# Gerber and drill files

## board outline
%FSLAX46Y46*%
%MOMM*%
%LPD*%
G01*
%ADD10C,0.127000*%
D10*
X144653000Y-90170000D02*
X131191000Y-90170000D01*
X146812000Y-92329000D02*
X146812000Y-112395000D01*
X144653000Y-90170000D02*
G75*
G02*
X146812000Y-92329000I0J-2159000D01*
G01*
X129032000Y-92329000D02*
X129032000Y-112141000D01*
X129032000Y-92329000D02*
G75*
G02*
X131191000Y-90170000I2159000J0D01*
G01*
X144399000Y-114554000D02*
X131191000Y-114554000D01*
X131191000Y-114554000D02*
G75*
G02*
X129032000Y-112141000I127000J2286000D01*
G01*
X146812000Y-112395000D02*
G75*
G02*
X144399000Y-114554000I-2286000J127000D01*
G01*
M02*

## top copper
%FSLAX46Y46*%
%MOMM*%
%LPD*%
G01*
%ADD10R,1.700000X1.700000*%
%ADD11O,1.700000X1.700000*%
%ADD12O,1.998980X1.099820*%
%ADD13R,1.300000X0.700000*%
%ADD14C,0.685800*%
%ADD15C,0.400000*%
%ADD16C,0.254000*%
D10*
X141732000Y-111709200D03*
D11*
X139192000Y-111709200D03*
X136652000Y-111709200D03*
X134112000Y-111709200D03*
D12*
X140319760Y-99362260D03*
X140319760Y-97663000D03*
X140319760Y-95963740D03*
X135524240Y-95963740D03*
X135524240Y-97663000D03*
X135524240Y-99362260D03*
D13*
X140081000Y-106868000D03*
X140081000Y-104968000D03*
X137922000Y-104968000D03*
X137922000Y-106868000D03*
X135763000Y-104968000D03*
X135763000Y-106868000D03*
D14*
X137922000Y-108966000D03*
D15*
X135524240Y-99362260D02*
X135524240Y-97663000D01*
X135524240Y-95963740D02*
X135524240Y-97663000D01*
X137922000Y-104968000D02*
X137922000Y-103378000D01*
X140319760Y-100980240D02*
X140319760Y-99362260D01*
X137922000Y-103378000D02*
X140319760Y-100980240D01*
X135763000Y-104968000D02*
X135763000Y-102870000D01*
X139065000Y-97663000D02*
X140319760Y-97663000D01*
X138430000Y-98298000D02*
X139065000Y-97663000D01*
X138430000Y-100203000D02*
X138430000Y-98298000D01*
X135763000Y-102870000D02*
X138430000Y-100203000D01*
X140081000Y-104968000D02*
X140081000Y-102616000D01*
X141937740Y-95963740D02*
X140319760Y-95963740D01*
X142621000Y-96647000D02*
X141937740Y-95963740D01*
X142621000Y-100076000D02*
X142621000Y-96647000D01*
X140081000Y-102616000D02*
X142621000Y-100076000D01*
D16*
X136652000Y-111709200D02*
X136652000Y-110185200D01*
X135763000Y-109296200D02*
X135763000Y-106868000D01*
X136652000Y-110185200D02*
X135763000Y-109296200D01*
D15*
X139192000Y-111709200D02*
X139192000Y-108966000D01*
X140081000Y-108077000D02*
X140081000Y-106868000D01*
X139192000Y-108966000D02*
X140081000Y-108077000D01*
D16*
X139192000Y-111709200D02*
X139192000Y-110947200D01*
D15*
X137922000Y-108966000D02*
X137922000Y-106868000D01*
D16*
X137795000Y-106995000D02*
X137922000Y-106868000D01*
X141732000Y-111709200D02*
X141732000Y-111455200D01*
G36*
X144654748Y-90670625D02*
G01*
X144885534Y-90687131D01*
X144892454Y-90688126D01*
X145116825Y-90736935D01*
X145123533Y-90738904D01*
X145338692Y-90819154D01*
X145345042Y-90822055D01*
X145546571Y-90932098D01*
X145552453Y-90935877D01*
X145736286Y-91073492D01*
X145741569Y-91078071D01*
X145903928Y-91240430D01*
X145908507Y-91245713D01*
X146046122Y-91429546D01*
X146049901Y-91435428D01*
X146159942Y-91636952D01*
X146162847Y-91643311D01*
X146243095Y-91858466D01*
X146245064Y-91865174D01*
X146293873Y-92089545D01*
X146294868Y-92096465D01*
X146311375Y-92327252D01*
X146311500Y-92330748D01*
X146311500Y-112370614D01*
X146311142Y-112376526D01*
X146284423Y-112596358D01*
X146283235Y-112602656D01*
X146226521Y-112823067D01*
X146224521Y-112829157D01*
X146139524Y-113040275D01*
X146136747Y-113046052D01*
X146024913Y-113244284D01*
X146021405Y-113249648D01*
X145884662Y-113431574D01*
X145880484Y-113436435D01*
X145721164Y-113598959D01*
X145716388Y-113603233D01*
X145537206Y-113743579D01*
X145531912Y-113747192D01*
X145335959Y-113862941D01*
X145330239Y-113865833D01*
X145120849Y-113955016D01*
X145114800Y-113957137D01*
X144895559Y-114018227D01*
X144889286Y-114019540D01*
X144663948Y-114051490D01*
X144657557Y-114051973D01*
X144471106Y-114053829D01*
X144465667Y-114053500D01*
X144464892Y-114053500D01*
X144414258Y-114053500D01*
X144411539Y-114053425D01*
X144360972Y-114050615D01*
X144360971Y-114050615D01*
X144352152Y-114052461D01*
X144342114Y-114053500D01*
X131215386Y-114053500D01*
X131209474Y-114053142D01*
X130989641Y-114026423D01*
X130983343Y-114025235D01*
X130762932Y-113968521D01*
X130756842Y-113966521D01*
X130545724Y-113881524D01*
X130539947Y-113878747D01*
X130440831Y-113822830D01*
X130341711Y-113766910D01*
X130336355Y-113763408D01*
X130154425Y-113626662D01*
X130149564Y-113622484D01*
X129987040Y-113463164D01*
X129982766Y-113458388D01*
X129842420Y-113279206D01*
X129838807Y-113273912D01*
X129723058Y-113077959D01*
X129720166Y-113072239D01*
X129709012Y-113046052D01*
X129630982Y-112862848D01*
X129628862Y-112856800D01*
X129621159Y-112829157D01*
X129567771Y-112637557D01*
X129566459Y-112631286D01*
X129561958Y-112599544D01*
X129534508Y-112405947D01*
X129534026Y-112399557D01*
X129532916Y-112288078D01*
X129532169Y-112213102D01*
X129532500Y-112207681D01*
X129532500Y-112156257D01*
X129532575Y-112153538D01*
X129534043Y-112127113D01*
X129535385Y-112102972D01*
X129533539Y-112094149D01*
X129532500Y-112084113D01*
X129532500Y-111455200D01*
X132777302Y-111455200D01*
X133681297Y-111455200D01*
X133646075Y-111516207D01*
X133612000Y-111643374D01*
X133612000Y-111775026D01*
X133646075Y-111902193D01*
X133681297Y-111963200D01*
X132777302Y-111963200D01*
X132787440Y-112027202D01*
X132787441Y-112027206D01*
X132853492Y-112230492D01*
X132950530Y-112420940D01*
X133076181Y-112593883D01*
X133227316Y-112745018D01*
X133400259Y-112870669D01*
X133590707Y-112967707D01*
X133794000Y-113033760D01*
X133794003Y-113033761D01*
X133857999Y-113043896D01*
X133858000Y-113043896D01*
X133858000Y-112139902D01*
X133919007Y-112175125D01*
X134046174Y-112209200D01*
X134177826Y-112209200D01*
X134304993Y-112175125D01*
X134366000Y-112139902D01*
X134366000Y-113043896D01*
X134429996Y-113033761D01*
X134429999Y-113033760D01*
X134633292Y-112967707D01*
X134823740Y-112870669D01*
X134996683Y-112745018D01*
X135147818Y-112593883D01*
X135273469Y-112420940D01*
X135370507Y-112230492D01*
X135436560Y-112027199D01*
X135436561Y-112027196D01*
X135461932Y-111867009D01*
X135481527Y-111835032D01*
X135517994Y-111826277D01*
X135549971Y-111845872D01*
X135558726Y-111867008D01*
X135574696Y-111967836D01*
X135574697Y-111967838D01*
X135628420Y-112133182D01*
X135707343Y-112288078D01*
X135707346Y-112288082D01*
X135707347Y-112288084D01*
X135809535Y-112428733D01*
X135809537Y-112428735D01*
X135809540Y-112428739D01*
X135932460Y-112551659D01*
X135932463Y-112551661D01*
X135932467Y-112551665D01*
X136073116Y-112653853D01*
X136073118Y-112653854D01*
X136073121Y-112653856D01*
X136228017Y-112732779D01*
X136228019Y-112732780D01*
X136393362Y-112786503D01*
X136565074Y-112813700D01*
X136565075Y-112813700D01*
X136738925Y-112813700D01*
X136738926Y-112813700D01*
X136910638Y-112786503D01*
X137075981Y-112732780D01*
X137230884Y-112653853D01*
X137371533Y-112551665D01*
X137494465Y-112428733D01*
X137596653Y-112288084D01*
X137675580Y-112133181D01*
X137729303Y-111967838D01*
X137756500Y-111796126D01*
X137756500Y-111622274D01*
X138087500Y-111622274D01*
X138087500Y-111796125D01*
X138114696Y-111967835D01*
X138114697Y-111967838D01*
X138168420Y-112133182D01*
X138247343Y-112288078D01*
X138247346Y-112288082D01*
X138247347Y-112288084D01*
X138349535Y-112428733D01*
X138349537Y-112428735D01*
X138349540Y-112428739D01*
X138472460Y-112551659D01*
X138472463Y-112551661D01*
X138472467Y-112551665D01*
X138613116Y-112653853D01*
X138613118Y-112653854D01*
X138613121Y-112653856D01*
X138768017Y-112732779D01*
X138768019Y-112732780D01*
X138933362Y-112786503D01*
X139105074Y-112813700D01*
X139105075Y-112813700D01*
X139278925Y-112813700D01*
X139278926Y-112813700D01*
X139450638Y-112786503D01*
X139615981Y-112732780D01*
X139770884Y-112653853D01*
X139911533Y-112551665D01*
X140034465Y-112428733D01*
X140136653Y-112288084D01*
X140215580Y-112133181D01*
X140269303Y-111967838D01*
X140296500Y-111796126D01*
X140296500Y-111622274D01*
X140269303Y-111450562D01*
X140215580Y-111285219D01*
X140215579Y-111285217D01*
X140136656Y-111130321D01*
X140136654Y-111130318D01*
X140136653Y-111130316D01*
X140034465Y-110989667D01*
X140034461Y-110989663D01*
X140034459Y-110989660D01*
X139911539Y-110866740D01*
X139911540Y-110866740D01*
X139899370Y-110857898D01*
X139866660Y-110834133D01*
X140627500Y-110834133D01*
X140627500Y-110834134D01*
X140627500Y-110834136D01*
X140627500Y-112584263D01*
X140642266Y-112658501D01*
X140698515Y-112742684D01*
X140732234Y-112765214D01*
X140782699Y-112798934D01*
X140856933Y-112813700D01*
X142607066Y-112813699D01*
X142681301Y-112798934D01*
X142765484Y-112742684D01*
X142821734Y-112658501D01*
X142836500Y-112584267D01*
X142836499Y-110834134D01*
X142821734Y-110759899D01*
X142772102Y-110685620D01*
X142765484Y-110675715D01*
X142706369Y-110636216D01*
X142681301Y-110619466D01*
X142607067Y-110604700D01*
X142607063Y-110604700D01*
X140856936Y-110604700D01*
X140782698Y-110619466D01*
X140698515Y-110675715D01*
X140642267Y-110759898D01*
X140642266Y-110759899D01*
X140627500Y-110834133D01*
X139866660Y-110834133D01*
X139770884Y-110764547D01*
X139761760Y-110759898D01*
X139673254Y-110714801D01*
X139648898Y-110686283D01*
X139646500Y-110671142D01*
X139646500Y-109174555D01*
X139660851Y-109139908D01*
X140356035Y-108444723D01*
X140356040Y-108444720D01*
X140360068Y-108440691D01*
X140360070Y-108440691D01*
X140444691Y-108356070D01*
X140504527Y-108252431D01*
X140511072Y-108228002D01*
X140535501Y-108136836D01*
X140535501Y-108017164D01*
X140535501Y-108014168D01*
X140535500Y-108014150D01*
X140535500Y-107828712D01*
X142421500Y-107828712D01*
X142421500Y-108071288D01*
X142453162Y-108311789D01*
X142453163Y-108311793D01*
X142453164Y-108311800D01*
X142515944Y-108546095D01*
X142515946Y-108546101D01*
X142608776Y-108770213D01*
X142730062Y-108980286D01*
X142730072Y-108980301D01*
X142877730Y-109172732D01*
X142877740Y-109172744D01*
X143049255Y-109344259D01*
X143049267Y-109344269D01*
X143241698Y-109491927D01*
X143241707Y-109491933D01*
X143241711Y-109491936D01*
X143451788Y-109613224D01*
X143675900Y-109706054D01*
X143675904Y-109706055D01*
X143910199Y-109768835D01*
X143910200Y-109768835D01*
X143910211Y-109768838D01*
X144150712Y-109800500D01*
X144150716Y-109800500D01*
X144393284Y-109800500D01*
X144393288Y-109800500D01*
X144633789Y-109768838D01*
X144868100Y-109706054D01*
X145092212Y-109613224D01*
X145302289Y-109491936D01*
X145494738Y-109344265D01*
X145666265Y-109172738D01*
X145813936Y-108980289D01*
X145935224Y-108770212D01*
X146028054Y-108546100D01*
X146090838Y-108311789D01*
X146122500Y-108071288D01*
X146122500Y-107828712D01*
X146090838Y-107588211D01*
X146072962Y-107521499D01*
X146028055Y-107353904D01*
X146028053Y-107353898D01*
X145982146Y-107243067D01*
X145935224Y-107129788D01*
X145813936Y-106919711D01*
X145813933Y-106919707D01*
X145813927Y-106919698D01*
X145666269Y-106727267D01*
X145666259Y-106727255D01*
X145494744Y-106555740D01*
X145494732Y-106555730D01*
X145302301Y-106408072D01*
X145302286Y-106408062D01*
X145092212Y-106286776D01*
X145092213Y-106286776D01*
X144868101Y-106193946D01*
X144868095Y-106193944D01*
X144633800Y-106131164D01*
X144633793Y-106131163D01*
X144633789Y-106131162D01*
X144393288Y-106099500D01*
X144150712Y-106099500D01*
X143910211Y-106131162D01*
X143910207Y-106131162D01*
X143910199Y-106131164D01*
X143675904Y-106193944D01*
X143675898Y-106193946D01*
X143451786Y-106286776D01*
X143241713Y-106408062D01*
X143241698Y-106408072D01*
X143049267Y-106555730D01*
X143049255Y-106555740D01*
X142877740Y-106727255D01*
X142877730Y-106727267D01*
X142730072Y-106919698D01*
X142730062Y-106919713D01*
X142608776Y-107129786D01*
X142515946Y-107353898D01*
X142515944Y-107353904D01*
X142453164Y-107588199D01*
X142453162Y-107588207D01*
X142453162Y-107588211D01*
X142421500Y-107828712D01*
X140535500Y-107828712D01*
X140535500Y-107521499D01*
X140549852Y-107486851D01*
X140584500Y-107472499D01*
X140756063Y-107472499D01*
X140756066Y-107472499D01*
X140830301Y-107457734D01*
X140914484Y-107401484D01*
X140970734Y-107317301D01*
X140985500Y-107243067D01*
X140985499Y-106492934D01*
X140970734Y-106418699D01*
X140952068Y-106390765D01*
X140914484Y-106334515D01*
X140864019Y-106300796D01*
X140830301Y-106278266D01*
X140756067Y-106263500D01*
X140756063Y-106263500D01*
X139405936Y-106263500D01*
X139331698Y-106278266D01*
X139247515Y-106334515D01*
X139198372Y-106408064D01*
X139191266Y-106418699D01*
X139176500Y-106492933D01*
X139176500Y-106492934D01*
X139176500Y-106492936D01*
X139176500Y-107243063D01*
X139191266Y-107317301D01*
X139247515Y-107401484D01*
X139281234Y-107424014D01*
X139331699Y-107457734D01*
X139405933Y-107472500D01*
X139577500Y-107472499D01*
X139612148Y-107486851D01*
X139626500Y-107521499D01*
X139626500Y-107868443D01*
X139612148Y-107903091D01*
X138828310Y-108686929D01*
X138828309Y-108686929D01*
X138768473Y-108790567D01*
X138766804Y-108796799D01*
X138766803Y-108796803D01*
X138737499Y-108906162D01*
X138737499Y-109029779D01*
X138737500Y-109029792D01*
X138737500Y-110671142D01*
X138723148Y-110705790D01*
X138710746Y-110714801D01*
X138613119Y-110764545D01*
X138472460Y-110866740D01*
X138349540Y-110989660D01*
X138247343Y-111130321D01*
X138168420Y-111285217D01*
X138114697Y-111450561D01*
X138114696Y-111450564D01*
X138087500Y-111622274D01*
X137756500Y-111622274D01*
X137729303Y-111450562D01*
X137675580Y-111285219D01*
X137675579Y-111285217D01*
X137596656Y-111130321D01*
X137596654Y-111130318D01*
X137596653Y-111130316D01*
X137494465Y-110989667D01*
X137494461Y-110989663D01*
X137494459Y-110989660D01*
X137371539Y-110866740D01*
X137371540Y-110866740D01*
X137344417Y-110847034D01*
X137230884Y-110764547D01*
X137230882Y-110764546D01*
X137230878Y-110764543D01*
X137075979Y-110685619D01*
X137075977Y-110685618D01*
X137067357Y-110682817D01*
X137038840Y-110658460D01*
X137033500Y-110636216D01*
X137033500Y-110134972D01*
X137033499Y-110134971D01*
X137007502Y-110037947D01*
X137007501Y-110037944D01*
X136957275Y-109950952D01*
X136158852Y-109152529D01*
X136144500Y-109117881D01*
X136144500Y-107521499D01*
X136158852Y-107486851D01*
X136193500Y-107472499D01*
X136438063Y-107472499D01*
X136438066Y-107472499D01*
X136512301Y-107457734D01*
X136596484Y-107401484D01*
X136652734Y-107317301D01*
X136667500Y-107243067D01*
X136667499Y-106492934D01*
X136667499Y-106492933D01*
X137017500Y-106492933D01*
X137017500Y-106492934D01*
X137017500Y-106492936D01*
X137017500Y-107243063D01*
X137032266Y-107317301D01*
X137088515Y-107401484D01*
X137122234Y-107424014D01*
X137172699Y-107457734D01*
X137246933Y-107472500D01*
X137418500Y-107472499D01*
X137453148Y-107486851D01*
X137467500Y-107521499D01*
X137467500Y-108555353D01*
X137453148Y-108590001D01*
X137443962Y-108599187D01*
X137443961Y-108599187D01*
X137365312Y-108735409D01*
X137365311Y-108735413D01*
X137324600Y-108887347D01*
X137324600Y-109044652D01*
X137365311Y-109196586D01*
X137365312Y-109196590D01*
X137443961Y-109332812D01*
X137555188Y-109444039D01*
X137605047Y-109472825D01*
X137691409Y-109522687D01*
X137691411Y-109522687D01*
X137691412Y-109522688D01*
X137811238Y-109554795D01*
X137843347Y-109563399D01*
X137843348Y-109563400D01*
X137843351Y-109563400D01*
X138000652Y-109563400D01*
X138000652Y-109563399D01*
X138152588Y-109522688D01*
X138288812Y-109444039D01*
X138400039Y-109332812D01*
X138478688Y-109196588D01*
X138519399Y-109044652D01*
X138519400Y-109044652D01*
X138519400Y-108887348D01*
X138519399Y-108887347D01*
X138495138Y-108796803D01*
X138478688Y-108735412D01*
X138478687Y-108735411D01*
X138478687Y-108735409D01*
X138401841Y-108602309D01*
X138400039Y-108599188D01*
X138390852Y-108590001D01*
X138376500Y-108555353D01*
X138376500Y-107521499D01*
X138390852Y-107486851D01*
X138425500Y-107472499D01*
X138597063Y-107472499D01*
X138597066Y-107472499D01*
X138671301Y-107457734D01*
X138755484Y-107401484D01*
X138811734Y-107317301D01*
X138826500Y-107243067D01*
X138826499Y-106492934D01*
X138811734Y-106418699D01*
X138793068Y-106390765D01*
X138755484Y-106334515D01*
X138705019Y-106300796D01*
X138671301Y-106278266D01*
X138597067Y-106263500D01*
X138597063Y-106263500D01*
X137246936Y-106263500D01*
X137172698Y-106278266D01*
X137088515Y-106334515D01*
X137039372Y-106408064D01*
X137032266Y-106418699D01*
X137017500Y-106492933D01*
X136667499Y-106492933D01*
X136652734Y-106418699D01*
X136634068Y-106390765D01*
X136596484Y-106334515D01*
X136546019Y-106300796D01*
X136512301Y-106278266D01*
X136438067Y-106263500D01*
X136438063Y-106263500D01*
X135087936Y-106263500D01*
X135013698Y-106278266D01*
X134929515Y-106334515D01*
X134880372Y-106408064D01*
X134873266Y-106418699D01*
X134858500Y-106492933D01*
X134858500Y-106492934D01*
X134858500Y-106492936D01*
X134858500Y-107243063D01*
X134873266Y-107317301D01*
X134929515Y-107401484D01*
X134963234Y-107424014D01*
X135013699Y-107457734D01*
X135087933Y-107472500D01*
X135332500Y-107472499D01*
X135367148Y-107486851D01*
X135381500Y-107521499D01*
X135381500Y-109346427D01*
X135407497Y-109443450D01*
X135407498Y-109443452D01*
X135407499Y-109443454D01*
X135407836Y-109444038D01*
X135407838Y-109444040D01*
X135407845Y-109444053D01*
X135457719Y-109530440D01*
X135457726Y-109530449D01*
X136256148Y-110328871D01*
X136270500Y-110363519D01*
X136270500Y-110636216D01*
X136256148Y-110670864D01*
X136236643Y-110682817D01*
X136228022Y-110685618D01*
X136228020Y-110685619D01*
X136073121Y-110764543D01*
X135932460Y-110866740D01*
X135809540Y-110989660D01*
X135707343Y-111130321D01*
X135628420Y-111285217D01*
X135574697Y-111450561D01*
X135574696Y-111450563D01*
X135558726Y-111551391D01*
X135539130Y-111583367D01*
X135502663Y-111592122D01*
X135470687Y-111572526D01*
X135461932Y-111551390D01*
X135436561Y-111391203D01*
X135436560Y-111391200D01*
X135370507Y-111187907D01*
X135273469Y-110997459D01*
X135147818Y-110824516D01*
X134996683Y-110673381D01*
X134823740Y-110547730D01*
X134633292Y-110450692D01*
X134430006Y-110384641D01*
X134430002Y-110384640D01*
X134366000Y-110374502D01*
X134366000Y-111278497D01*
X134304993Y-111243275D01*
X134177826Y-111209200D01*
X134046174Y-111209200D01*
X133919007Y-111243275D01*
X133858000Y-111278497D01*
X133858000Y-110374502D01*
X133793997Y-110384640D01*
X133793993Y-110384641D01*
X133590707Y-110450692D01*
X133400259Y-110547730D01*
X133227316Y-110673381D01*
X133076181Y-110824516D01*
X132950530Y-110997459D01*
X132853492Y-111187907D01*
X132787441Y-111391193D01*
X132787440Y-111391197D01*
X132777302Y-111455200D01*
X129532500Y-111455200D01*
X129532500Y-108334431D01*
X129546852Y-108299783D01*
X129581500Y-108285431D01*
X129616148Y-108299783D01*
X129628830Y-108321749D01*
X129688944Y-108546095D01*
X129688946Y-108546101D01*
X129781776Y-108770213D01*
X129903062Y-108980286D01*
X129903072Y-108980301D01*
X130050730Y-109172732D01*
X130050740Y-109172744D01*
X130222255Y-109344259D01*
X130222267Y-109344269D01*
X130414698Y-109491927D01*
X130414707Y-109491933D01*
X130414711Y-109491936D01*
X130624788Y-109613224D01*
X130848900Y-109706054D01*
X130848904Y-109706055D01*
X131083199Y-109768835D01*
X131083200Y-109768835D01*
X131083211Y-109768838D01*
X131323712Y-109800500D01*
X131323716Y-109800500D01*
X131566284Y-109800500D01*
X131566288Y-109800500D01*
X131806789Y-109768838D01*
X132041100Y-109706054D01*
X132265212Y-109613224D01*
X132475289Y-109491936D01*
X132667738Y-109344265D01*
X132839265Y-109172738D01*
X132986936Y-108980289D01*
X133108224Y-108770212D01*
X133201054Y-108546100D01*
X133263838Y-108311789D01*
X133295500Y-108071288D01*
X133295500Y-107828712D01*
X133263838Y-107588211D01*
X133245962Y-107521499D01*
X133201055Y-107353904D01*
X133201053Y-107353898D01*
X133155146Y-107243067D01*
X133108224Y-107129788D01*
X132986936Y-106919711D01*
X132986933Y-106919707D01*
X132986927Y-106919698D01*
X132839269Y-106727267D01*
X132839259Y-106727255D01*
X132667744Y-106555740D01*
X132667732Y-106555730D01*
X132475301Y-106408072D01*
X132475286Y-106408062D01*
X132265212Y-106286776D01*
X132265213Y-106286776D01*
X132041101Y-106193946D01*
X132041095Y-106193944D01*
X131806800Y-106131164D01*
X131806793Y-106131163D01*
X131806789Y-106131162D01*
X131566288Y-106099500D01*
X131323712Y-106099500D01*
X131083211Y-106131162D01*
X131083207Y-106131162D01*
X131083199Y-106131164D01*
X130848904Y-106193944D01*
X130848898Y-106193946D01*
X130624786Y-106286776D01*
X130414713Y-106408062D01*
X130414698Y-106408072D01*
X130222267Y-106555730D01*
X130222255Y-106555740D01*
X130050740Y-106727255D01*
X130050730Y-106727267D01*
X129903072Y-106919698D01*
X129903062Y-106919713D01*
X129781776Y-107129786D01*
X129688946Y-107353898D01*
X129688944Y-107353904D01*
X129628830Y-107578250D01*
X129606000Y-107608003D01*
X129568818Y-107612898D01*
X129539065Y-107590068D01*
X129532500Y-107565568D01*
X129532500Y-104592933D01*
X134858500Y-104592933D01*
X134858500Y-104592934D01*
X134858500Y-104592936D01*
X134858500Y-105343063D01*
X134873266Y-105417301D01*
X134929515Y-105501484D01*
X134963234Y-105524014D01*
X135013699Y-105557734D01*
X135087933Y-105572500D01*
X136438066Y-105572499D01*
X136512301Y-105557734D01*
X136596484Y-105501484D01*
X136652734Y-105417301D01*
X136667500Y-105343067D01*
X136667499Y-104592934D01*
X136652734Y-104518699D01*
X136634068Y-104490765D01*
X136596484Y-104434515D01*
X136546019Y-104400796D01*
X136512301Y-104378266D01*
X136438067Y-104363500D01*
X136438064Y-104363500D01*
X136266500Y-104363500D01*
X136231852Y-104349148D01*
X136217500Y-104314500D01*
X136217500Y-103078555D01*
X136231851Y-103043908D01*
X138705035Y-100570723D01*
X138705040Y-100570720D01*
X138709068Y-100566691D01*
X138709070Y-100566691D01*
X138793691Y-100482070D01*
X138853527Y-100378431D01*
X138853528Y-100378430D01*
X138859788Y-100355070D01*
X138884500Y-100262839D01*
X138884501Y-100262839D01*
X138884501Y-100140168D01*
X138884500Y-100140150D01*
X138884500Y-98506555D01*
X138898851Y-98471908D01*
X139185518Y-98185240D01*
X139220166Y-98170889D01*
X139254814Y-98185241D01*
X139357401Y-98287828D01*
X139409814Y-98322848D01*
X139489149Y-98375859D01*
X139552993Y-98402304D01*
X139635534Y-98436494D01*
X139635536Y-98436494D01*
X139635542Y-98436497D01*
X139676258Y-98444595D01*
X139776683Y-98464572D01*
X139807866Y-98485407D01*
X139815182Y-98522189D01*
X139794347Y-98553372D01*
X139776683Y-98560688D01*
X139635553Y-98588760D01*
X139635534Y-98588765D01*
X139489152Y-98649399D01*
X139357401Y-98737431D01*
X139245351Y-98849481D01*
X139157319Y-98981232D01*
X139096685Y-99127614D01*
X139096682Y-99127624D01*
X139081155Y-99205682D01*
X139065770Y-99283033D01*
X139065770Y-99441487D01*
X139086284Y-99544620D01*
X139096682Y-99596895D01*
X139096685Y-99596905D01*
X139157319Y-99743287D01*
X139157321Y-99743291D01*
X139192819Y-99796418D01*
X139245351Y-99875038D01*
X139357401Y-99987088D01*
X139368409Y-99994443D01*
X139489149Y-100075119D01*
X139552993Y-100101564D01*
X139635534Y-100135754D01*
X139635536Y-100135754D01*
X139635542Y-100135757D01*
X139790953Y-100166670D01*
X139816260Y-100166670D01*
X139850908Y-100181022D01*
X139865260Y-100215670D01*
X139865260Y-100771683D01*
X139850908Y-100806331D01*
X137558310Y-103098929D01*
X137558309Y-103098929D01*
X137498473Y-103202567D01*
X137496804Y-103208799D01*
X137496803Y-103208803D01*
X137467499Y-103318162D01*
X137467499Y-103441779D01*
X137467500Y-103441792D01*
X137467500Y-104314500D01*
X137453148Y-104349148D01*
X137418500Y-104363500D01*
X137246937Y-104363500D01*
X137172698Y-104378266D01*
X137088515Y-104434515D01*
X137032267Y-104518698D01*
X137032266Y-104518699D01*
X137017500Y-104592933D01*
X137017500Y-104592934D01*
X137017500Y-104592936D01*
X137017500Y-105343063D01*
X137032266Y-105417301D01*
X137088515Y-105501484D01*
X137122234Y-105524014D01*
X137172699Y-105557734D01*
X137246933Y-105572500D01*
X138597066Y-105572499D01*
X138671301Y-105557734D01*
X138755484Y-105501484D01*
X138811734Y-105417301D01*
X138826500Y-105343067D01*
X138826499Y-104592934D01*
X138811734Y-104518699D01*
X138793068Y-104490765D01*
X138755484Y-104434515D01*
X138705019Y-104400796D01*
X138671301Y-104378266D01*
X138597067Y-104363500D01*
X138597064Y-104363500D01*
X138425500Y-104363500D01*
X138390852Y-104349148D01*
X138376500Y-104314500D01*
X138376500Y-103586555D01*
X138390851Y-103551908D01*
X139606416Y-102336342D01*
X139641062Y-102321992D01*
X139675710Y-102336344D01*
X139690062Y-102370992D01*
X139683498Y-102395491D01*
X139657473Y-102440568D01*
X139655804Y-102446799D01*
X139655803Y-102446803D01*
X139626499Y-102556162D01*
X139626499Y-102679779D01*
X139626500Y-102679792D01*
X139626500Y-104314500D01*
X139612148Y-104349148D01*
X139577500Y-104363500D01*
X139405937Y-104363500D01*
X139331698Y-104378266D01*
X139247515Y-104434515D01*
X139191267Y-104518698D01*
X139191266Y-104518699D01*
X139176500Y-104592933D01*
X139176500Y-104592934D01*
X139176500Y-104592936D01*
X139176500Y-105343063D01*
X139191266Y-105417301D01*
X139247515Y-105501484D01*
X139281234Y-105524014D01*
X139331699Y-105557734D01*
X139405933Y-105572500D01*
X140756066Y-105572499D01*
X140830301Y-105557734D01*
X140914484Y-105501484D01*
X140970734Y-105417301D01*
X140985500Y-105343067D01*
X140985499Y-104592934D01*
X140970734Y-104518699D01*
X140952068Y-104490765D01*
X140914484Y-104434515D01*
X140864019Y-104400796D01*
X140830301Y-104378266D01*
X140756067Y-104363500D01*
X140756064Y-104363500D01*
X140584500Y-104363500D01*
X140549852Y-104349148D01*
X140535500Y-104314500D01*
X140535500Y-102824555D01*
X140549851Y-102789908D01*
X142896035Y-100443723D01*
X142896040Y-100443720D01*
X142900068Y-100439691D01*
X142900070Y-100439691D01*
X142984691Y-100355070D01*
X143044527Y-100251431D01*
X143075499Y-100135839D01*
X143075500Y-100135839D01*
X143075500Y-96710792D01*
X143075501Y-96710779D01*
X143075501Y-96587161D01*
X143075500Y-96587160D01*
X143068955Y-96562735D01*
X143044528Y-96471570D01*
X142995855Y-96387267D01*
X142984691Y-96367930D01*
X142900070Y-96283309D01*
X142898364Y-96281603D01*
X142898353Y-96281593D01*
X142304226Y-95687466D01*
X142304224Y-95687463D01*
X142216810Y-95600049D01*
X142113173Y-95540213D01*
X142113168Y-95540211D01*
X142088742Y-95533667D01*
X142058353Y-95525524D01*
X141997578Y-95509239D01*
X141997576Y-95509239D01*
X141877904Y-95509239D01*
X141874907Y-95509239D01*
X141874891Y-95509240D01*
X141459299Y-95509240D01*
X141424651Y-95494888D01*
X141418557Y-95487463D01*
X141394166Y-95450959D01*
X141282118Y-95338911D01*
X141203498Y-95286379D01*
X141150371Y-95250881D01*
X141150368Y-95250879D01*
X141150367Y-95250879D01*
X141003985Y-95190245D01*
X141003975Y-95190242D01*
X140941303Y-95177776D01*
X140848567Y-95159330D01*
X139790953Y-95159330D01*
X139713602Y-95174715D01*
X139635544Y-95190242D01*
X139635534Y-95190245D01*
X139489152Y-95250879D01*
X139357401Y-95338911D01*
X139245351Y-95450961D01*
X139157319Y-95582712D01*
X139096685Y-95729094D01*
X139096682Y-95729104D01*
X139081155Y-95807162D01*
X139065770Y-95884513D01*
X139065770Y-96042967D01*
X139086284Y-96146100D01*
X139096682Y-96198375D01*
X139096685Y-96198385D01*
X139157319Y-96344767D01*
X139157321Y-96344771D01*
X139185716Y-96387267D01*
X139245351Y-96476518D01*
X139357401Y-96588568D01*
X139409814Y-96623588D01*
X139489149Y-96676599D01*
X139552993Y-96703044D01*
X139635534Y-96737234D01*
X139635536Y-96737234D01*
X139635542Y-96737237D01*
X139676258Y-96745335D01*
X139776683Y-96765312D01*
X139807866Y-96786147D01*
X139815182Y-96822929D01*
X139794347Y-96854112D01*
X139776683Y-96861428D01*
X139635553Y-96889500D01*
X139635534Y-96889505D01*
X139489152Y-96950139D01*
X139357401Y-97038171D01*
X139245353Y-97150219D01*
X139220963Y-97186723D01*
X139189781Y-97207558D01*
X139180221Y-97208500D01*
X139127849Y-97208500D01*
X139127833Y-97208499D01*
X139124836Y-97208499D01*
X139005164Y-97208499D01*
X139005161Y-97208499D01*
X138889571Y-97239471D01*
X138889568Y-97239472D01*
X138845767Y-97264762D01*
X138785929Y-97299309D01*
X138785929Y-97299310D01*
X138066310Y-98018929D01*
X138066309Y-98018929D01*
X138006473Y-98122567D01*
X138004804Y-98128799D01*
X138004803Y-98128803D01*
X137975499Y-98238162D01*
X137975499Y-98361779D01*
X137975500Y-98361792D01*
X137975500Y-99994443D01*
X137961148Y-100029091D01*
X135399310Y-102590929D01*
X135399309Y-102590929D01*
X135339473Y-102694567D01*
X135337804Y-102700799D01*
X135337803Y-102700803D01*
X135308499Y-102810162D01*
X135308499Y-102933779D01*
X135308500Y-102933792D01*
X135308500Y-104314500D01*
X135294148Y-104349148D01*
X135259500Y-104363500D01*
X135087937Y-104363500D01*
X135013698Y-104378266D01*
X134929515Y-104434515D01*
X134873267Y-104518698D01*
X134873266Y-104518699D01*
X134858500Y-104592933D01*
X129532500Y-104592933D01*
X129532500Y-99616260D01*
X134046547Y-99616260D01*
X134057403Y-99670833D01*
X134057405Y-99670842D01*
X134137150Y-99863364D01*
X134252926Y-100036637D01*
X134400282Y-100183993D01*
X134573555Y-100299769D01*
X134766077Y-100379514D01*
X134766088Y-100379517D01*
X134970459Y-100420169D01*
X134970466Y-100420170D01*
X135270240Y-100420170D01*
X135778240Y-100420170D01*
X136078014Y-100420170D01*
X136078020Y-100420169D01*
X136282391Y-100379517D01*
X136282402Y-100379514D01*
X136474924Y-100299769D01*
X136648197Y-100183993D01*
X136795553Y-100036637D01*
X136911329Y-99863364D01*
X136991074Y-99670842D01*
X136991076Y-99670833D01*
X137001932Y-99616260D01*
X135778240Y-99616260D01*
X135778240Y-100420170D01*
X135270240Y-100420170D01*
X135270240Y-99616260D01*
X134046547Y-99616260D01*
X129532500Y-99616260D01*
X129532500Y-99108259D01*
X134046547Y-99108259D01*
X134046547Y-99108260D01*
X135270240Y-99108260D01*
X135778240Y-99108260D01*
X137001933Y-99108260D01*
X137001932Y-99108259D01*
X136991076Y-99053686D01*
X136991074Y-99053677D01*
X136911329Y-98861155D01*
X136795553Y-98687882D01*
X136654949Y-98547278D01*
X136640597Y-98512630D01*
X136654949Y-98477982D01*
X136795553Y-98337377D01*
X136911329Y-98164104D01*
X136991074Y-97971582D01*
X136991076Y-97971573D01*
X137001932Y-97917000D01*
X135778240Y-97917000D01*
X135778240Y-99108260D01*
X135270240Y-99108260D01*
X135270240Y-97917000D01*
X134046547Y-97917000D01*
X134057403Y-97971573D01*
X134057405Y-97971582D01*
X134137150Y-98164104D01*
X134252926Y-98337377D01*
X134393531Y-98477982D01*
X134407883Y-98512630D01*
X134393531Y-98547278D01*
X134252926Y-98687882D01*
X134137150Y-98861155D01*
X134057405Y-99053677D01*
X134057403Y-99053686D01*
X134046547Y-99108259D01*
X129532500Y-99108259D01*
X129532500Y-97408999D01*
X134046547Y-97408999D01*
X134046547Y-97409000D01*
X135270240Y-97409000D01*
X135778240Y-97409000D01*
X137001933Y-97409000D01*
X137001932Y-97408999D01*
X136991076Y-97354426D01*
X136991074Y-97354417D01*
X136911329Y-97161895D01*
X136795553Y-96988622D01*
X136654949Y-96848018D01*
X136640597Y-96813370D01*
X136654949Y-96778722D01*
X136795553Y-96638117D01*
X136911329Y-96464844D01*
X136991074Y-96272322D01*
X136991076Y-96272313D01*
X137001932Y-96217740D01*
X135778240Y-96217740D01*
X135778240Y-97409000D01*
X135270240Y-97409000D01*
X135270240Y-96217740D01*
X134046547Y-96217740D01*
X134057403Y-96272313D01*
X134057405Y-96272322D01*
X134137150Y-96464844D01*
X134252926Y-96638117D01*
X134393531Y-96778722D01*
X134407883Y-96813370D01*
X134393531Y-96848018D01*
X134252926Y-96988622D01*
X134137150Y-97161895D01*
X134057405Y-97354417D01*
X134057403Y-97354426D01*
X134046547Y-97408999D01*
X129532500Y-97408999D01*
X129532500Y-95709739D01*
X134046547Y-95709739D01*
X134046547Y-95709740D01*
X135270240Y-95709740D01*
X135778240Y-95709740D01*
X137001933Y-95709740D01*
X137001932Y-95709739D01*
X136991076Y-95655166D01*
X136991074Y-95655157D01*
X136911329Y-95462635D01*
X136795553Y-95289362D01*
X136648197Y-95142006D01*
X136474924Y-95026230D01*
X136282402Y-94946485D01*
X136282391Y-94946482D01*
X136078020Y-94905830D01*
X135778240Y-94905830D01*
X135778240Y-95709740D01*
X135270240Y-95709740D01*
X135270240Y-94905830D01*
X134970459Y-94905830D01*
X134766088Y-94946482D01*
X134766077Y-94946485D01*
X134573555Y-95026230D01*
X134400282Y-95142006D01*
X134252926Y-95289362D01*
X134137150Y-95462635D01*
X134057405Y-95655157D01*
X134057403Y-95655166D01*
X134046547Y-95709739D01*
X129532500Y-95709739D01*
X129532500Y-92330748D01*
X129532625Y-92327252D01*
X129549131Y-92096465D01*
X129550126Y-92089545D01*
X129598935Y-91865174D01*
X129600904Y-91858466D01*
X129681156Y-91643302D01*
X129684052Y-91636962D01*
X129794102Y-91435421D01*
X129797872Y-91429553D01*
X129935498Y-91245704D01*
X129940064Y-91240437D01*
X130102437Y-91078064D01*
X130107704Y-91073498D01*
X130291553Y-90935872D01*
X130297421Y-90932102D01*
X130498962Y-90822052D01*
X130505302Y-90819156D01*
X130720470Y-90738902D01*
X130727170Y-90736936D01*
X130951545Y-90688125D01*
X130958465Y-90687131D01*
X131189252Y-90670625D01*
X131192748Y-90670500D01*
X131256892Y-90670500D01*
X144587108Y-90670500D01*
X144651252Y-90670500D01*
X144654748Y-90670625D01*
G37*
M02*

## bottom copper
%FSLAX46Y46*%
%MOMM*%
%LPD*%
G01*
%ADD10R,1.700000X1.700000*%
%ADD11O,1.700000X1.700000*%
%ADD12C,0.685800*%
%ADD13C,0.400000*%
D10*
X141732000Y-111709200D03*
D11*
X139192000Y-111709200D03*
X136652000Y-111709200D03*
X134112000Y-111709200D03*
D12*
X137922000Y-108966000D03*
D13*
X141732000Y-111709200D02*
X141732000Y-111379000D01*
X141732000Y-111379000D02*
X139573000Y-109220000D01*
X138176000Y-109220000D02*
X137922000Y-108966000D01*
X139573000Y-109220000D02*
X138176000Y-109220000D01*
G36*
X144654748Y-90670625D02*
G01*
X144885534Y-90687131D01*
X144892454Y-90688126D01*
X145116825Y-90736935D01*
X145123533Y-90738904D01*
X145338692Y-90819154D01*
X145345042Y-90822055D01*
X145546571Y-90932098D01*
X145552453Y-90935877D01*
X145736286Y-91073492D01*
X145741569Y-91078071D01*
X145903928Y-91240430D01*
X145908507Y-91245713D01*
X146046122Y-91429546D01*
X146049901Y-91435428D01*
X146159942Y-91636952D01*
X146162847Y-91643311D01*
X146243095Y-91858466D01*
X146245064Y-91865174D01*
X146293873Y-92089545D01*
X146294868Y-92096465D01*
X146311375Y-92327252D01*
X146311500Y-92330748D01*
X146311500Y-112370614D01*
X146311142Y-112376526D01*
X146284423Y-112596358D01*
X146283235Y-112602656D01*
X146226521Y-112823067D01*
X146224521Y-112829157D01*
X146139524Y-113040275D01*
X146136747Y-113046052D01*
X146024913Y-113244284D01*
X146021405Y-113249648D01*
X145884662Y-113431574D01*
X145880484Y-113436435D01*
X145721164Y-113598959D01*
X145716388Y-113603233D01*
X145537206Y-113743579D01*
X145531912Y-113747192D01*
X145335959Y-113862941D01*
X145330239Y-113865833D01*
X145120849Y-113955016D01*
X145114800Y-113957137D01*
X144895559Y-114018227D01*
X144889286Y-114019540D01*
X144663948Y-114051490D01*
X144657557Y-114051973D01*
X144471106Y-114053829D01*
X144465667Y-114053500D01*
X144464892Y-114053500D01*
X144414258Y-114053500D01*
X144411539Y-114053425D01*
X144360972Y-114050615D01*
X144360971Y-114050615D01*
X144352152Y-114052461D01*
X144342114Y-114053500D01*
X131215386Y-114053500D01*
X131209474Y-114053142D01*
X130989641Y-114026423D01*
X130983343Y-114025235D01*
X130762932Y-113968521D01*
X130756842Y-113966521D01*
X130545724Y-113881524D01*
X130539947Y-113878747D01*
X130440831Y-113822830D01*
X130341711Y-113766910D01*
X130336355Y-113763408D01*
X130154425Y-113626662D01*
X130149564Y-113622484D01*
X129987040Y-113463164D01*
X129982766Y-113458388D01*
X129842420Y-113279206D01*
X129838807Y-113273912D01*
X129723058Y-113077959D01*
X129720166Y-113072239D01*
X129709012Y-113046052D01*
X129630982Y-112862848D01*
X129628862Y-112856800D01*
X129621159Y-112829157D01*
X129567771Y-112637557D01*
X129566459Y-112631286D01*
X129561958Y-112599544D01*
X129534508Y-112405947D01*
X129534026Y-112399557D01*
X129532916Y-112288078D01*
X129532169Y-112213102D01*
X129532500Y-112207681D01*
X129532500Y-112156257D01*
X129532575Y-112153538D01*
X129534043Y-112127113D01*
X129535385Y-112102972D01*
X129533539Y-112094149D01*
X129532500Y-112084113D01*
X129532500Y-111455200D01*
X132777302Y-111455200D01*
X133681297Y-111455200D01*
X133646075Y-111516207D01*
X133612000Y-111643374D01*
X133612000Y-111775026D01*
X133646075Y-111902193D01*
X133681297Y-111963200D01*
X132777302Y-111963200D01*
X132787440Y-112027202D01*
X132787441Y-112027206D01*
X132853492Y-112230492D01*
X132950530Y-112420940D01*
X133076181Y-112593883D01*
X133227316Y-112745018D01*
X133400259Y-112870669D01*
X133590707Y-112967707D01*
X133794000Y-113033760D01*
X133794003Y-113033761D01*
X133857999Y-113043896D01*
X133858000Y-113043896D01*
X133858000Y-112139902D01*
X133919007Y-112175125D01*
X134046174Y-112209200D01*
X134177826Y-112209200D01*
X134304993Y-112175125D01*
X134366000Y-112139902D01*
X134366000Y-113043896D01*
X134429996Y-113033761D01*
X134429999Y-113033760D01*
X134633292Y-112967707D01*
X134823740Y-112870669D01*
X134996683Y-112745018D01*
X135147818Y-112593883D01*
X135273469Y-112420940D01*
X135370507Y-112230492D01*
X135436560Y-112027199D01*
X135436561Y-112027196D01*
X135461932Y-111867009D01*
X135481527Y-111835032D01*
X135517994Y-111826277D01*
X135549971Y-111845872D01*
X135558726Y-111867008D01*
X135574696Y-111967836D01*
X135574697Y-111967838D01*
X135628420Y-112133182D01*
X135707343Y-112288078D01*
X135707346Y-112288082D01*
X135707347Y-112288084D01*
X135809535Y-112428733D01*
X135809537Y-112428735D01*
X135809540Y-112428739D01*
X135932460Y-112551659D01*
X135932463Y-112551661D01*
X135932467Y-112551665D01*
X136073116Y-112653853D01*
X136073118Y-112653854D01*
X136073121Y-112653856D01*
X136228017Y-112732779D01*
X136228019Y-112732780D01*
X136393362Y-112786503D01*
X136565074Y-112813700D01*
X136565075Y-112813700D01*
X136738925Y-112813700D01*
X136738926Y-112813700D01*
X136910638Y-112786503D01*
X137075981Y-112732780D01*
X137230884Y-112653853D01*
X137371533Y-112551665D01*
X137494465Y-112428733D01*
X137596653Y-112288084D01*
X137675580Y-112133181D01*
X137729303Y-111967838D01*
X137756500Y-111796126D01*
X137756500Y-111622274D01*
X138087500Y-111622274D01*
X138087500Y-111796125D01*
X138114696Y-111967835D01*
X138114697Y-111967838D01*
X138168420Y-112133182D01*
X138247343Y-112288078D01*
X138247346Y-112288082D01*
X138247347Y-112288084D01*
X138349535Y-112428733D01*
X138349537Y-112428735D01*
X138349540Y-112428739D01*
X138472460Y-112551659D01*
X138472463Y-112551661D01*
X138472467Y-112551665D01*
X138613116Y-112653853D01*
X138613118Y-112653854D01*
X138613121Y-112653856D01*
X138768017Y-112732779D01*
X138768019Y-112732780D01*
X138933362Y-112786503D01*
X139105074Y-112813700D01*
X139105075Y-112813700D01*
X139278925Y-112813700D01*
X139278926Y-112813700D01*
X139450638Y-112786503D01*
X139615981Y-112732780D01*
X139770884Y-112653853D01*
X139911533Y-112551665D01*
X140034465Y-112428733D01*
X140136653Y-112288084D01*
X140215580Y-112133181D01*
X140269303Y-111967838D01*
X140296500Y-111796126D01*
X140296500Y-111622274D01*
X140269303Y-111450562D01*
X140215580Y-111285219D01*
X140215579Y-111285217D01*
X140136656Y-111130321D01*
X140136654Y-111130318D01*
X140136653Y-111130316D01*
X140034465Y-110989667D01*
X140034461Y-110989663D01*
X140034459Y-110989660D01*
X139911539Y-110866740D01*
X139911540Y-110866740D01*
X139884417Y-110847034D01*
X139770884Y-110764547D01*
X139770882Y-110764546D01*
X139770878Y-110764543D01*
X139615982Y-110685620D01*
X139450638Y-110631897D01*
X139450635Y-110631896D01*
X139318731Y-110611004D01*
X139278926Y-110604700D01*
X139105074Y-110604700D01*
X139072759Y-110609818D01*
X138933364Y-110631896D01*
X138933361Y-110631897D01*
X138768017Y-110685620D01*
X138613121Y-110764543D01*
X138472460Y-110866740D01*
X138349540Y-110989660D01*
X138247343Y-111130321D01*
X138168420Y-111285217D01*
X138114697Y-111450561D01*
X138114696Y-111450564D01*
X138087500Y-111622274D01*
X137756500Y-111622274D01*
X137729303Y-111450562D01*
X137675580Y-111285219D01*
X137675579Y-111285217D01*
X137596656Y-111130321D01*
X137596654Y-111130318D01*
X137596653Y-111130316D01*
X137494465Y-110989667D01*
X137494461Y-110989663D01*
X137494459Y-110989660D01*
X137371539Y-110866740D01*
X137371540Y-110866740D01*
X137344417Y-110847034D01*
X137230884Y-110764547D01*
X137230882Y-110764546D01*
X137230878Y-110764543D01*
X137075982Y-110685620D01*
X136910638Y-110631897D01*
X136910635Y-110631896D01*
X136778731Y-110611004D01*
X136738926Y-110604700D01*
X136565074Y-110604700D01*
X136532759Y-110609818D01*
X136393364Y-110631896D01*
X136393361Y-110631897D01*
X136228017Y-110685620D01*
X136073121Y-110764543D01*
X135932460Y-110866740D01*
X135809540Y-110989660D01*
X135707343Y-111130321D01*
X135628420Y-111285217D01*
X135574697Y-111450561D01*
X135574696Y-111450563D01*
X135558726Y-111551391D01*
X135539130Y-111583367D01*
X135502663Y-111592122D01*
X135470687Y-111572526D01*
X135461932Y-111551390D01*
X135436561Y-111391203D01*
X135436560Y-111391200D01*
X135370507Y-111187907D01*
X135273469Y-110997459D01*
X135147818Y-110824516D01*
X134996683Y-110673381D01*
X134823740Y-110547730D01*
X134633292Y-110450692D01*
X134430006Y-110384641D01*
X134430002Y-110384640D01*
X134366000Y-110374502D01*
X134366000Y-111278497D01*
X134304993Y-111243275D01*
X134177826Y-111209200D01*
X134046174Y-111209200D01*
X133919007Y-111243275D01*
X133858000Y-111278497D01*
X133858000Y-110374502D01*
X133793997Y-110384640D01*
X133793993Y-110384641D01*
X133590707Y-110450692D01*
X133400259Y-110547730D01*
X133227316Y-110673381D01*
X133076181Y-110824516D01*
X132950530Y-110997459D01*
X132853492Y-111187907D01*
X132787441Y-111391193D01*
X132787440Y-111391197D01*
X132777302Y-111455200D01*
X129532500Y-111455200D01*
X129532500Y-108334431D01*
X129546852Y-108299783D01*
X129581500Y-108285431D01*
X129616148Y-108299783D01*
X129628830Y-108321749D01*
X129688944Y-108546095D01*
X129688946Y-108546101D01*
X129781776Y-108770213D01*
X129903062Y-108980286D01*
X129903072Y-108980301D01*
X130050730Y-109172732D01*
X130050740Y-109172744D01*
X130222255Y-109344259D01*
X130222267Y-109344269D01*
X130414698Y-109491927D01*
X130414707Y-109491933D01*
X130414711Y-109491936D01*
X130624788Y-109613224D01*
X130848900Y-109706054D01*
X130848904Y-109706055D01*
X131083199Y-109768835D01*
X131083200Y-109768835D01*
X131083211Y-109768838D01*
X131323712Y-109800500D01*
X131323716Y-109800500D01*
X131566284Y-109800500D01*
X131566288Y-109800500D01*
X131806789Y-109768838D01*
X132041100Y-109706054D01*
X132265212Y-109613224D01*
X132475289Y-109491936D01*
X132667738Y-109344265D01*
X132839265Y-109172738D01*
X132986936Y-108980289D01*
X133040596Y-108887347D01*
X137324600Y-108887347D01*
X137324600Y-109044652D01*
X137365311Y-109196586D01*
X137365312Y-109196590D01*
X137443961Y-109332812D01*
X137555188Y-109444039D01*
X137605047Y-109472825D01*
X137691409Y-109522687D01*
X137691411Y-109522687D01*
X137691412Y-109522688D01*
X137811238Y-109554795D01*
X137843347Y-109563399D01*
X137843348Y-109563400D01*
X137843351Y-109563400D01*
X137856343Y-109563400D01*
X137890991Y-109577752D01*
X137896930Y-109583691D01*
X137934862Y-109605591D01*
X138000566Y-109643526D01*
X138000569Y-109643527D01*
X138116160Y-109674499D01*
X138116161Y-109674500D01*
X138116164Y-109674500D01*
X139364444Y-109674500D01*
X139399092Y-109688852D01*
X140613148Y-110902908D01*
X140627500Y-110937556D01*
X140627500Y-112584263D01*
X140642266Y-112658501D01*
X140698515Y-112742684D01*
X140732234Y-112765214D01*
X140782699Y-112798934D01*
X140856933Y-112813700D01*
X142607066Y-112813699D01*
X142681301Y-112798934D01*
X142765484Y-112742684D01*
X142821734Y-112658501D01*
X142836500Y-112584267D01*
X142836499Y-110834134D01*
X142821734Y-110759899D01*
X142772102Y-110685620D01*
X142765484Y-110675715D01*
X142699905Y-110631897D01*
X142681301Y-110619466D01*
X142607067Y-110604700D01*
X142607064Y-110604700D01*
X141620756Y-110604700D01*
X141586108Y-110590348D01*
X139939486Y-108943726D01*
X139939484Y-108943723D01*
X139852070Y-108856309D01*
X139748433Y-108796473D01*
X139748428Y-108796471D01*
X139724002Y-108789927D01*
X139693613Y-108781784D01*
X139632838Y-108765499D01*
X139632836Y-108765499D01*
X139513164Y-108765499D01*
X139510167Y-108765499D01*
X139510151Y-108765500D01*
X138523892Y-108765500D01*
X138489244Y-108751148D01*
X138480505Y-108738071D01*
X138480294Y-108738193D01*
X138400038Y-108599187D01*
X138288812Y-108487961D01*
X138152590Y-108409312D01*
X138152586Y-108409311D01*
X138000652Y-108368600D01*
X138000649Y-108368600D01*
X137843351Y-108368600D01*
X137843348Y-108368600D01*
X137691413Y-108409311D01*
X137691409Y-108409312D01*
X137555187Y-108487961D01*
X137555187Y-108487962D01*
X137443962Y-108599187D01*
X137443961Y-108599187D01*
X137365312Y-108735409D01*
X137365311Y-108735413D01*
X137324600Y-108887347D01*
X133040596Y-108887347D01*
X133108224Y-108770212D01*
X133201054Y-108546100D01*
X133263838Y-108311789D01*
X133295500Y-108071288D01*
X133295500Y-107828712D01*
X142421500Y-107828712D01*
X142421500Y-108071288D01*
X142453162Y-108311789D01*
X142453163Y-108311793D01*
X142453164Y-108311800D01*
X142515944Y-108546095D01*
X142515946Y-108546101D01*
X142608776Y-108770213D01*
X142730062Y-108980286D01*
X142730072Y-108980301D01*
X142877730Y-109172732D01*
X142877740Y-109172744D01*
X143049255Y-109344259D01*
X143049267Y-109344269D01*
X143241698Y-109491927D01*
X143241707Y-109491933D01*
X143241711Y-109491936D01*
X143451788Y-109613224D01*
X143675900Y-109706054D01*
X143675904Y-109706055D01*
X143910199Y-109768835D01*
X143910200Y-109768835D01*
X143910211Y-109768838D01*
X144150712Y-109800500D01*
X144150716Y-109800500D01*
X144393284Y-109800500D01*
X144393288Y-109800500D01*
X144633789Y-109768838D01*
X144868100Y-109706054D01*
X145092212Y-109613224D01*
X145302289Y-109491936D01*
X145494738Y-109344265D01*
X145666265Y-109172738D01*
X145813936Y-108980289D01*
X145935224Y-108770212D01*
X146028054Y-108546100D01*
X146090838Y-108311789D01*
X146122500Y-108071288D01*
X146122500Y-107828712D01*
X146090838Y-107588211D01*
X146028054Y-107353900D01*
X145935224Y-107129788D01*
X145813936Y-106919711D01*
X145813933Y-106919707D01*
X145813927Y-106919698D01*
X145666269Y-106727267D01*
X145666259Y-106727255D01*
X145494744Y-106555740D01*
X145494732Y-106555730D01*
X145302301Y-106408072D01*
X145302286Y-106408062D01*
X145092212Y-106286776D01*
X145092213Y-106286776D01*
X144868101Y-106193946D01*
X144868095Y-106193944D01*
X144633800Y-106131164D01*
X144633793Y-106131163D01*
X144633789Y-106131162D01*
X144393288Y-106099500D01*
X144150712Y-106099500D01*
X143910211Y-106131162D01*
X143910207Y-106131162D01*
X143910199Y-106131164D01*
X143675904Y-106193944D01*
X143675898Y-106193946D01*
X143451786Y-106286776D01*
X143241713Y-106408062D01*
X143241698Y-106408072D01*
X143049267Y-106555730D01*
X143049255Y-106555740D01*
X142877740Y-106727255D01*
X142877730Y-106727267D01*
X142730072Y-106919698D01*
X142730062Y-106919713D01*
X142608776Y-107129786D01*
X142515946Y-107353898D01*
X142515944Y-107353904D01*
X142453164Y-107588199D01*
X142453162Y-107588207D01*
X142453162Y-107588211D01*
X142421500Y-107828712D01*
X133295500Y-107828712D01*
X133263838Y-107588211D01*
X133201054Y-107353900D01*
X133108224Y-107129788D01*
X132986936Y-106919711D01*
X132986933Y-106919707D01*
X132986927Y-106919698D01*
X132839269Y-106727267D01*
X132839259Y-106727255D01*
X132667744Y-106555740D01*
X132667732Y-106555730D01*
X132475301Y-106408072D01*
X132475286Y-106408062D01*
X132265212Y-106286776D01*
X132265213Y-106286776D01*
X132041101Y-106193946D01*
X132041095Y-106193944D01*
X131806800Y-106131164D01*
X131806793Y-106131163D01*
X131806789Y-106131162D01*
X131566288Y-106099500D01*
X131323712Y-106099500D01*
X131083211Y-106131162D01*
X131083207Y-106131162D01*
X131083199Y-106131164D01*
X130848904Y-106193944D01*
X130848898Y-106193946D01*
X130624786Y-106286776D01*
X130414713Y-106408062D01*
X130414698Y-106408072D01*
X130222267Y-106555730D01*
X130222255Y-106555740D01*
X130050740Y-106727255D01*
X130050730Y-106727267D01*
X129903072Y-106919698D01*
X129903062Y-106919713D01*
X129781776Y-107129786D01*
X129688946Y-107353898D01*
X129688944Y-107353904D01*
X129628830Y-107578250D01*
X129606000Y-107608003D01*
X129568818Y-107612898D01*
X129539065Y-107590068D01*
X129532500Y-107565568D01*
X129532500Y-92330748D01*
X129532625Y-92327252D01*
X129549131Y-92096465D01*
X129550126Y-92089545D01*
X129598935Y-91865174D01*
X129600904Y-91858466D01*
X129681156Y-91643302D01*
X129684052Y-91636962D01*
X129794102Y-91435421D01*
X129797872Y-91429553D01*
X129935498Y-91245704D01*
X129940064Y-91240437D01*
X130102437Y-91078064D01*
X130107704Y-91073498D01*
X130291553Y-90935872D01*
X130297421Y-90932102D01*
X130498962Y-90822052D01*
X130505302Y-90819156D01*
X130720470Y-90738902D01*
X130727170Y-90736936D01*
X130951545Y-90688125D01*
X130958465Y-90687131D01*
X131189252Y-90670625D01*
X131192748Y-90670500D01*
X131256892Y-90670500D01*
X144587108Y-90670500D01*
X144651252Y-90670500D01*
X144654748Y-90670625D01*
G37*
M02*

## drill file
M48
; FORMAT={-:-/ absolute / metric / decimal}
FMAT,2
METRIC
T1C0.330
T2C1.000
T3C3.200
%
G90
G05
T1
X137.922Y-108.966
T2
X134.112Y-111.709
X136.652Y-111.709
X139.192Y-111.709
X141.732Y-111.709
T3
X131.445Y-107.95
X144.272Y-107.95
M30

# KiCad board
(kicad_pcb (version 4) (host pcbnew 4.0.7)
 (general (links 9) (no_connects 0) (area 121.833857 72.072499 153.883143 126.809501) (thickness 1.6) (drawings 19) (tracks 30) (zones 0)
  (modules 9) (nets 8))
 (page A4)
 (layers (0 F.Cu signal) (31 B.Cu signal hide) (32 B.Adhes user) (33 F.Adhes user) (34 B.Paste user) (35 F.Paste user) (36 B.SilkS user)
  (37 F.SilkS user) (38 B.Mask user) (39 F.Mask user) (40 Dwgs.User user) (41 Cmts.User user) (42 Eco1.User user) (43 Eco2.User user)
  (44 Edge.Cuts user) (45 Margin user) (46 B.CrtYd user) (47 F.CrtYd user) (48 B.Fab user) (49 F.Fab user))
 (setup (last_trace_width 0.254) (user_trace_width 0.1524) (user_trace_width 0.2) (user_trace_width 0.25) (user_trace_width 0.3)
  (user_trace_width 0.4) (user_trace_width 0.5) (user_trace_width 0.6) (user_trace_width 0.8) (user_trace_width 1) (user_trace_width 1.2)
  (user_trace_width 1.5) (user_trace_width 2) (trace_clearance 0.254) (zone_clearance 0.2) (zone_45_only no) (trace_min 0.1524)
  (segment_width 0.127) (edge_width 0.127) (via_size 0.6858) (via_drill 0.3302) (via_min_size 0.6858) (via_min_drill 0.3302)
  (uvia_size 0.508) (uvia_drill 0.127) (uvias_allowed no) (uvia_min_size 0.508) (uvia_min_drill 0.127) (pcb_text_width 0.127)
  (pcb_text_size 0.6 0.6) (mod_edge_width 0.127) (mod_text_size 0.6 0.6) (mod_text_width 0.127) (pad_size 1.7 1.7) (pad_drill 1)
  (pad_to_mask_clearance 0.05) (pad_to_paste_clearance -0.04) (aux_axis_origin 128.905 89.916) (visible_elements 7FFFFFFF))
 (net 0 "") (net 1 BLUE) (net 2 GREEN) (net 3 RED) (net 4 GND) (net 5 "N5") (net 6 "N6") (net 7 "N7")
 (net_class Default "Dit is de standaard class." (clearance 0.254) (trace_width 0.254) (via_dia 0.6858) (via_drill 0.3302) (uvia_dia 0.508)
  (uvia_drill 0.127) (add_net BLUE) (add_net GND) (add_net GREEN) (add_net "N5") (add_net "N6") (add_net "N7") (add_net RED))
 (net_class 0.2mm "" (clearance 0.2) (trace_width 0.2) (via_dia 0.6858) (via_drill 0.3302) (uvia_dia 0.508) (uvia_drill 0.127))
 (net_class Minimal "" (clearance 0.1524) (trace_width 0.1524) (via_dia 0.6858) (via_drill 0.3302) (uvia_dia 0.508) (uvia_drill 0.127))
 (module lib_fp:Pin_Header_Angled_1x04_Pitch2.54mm (layer F.Cu) (at 141.732 111.7092 270)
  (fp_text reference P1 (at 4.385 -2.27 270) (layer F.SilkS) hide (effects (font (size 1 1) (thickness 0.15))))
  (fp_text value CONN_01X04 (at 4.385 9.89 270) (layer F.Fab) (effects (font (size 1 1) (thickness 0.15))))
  (pad 4 thru_hole rect (at 0 0 270) (size 1.7 1.7) (drill 1) (layers *.Cu *.Mask) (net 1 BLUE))
  (pad 3 thru_hole oval (at 0 2.54 270) (size 1.7 1.7) (drill 1) (layers *.Cu *.Mask) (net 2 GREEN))
  (pad 2 thru_hole oval (at 0 5.08 270) (size 1.7 1.7) (drill 1) (layers *.Cu *.Mask) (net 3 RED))
  (pad 1 thru_hole oval (at 0 7.62 270) (size 1.7 1.7) (drill 1) (layers *.Cu *.Mask) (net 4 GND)))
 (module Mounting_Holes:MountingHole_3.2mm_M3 (layer F.Cu) (at 144.272 107.95)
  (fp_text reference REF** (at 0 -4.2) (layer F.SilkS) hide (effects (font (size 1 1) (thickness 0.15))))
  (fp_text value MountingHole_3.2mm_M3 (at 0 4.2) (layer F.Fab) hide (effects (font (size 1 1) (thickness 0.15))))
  (pad 1 np_thru_hole circle (at 0 0) (size 3.2 3.2) (drill 3.2) (layers *.Cu *.Mask)))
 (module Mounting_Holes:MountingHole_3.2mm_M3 (layer F.Cu) (at 131.445 107.95)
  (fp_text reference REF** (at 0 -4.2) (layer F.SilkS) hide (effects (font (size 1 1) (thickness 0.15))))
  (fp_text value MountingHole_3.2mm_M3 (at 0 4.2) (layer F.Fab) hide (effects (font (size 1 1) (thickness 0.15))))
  (pad 1 np_thru_hole circle (at 0 0) (size 3.2 3.2) (drill 3.2) (layers *.Cu *.Mask)))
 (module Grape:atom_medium (layer B.Cu) (at 137.922 97.6884 180)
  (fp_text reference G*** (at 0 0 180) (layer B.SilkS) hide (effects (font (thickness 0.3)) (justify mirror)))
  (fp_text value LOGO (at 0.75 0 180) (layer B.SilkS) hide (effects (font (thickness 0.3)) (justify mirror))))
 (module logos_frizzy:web (layer B.Cu) (at 137.8712 104.5972 180)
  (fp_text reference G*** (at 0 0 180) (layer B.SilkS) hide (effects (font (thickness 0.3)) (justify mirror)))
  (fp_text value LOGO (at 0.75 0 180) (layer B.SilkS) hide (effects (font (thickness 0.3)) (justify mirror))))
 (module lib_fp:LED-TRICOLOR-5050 (layer F.Cu) (at 137.922 97.663 180)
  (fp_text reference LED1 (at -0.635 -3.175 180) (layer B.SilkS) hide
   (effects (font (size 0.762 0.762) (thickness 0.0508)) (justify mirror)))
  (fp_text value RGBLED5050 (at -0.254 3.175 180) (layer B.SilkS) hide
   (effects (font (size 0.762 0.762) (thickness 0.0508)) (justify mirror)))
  (pad 1 smd oval (at -2.39776 -1.69926 180) (size 1.99898 1.09982) (layers F.Cu F.Paste F.Mask) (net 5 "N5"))
  (pad 2 smd oval (at -2.39776 0 180) (size 1.99898 1.09982) (layers F.Cu F.Paste F.Mask) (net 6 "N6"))
  (pad 3 smd oval (at -2.39776 1.69926 180) (size 1.99898 1.09982) (layers F.Cu F.Paste F.Mask) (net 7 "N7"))
  (pad 4 smd oval (at 2.39776 1.69926 180) (size 1.99898 1.09982) (layers F.Cu F.Paste F.Mask) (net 4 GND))
  (pad 5 smd oval (at 2.39776 0 180) (size 1.99898 1.09982) (layers F.Cu F.Paste F.Mask) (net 4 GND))
  (pad 6 smd oval (at 2.39776 -1.69926 180) (size 1.99898 1.09982) (layers F.Cu F.Paste F.Mask) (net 4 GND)))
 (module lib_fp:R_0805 (layer F.Cu) (at 140.081 105.918 90)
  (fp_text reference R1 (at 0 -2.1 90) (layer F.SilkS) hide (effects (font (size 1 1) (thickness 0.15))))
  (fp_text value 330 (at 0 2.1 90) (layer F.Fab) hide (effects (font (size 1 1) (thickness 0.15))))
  (pad 1 smd rect (at -0.95 0 90) (size 0.7 1.3) (layers F.Cu F.Paste F.Mask) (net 2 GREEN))
  (pad 2 smd rect (at 0.95 0 90) (size 0.7 1.3) (layers F.Cu F.Paste F.Mask) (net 7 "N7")))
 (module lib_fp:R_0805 (layer F.Cu) (at 137.922 105.918 270)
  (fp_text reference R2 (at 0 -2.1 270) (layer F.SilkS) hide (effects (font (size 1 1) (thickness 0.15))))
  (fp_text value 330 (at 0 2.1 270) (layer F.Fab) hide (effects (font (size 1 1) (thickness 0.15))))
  (pad 1 smd rect (at -0.95 0 270) (size 0.7 1.3) (layers F.Cu F.Paste F.Mask) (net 5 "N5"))
  (pad 2 smd rect (at 0.95 0 270) (size 0.7 1.3) (layers F.Cu F.Paste F.Mask) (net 1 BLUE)))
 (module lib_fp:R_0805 (layer F.Cu) (at 135.763 105.918 270)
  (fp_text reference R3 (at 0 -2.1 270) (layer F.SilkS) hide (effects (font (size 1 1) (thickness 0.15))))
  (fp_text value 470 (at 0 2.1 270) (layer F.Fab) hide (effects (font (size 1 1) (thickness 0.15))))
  (pad 1 smd rect (at -0.95 0 270) (size 0.7 1.3) (layers F.Cu F.Paste F.Mask) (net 6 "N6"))
  (pad 2 smd rect (at 0.95 0 270) (size 0.7 1.3) (layers F.Cu F.Paste F.Mask) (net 3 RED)))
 (gr_line (start 144.653 90.17) (end 131.191 90.17) (angle 90) (layer Edge.Cuts) (width 0.127))
 (gr_line (start 146.812 92.329) (end 146.812 112.395) (angle 90) (layer Edge.Cuts) (width 0.127))
 (gr_arc (start 144.653 92.329) (end 144.653 90.17) (angle 90) (layer Edge.Cuts) (width 0.127))
 (gr_line (start 129.032 92.329) (end 129.032 112.141) (angle 90) (layer Edge.Cuts) (width 0.127))
 (gr_arc (start 131.191 92.329) (end 129.032 92.329) (angle 90) (layer Edge.Cuts) (width 0.127))
 (gr_line (start 144.399 114.554) (end 131.191 114.554) (angle 90) (layer Edge.Cuts) (width 0.127))
 (gr_arc (start 131.318 112.268) (end 131.191 114.554) (angle 90) (layer Edge.Cuts) (width 0.127))
 (gr_arc (start 144.526 112.268) (end 146.812 112.395) (angle 90) (layer Edge.Cuts) (width 0.127))
 (segment (start 135.52424 99.36226) (end 135.52424 97.663) (width 0.4) (layer F.Cu) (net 4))
 (segment (start 135.52424 95.96374) (end 135.52424 97.663) (width 0.4) (layer F.Cu) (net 4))
 (segment (start 137.922 104.968) (end 137.922 103.378) (width 0.4) (layer F.Cu) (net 5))
 (segment (start 140.31976 100.98024) (end 140.31976 99.36226) (width 0.4) (layer F.Cu) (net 5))
 (segment (start 137.922 103.378) (end 140.31976 100.98024) (width 0.4) (layer F.Cu) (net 5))
 (segment (start 135.763 104.968) (end 135.763 102.87) (width 0.4) (layer F.Cu) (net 6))
 (segment (start 139.065 97.663) (end 140.31976 97.663) (width 0.4) (layer F.Cu) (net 6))
 (segment (start 138.43 98.298) (end 139.065 97.663) (width 0.4) (layer F.Cu) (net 6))
 (segment (start 138.43 100.203) (end 138.43 98.298) (width 0.4) (layer F.Cu) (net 6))
 (segment (start 135.763 102.87) (end 138.43 100.203) (width 0.4) (layer F.Cu) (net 6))
 (segment (start 140.081 104.968) (end 140.081 102.616) (width 0.4) (layer F.Cu) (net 7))
 (segment (start 141.93774 95.96374) (end 140.31976 95.96374) (width 0.4) (layer F.Cu) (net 7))
 (segment (start 142.621 96.647) (end 141.93774 95.96374) (width 0.4) (layer F.Cu) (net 7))
 (segment (start 142.621 100.076) (end 142.621 96.647) (width 0.4) (layer F.Cu) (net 7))
 (segment (start 140.081 102.616) (end 142.621 100.076) (width 0.4) (layer F.Cu) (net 7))
 (segment (start 136.652 111.7092) (end 136.652 110.1852) (width 0.254) (layer F.Cu) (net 3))
 (segment (start 135.763 109.2962) (end 135.763 106.868) (width 0.254) (layer F.Cu) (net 3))
 (segment (start 136.652 110.1852) (end 135.763 109.2962) (width 0.254) (layer F.Cu) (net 3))
 (segment (start 139.192 111.7092) (end 139.192 108.966) (width 0.4) (layer F.Cu) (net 2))
 (segment (start 140.081 108.077) (end 140.081 106.868) (width 0.4) (layer F.Cu) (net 2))
 (segment (start 139.192 108.966) (end 140.081 108.077) (width 0.4) (layer F.Cu) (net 2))
 (segment (start 139.192 111.7092) (end 139.192 110.9472) (width 0.254) (layer F.Cu) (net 2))
 (segment (start 141.732 111.7092) (end 141.732 111.379) (width 0.4) (layer B.Cu) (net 1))
 (segment (start 141.732 111.379) (end 139.573 109.22) (width 0.4) (layer B.Cu) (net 1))
 (segment (start 137.922 108.966) (end 137.922 106.868) (width 0.4) (layer F.Cu) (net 1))
 (via (at 137.922 108.966) (size 0.6858) (drill 0.3302) (layers F.Cu B.Cu) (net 1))
 (segment (start 138.176 109.22) (end 137.922 108.966) (width 0.4) (layer B.Cu) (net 1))
 (segment (start 139.573 109.22) (end 138.176 109.22) (width 0.4) (layer B.Cu) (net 1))
 (segment (start 137.795 106.995) (end 137.922 106.868) (width 0.254) (layer F.Cu) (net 1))
 (segment (start 141.732 111.7092) (end 141.732 111.4552) (width 0.254) (layer F.Cu) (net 1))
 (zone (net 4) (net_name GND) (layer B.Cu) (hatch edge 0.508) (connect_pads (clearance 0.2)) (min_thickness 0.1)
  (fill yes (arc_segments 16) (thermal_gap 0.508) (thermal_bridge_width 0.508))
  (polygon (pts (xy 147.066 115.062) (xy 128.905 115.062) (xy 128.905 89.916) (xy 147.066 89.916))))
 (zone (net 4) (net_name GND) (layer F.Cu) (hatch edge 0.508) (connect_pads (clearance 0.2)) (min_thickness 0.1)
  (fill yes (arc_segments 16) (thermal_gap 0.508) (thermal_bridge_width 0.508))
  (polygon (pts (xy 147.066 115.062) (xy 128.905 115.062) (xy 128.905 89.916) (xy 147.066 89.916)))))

